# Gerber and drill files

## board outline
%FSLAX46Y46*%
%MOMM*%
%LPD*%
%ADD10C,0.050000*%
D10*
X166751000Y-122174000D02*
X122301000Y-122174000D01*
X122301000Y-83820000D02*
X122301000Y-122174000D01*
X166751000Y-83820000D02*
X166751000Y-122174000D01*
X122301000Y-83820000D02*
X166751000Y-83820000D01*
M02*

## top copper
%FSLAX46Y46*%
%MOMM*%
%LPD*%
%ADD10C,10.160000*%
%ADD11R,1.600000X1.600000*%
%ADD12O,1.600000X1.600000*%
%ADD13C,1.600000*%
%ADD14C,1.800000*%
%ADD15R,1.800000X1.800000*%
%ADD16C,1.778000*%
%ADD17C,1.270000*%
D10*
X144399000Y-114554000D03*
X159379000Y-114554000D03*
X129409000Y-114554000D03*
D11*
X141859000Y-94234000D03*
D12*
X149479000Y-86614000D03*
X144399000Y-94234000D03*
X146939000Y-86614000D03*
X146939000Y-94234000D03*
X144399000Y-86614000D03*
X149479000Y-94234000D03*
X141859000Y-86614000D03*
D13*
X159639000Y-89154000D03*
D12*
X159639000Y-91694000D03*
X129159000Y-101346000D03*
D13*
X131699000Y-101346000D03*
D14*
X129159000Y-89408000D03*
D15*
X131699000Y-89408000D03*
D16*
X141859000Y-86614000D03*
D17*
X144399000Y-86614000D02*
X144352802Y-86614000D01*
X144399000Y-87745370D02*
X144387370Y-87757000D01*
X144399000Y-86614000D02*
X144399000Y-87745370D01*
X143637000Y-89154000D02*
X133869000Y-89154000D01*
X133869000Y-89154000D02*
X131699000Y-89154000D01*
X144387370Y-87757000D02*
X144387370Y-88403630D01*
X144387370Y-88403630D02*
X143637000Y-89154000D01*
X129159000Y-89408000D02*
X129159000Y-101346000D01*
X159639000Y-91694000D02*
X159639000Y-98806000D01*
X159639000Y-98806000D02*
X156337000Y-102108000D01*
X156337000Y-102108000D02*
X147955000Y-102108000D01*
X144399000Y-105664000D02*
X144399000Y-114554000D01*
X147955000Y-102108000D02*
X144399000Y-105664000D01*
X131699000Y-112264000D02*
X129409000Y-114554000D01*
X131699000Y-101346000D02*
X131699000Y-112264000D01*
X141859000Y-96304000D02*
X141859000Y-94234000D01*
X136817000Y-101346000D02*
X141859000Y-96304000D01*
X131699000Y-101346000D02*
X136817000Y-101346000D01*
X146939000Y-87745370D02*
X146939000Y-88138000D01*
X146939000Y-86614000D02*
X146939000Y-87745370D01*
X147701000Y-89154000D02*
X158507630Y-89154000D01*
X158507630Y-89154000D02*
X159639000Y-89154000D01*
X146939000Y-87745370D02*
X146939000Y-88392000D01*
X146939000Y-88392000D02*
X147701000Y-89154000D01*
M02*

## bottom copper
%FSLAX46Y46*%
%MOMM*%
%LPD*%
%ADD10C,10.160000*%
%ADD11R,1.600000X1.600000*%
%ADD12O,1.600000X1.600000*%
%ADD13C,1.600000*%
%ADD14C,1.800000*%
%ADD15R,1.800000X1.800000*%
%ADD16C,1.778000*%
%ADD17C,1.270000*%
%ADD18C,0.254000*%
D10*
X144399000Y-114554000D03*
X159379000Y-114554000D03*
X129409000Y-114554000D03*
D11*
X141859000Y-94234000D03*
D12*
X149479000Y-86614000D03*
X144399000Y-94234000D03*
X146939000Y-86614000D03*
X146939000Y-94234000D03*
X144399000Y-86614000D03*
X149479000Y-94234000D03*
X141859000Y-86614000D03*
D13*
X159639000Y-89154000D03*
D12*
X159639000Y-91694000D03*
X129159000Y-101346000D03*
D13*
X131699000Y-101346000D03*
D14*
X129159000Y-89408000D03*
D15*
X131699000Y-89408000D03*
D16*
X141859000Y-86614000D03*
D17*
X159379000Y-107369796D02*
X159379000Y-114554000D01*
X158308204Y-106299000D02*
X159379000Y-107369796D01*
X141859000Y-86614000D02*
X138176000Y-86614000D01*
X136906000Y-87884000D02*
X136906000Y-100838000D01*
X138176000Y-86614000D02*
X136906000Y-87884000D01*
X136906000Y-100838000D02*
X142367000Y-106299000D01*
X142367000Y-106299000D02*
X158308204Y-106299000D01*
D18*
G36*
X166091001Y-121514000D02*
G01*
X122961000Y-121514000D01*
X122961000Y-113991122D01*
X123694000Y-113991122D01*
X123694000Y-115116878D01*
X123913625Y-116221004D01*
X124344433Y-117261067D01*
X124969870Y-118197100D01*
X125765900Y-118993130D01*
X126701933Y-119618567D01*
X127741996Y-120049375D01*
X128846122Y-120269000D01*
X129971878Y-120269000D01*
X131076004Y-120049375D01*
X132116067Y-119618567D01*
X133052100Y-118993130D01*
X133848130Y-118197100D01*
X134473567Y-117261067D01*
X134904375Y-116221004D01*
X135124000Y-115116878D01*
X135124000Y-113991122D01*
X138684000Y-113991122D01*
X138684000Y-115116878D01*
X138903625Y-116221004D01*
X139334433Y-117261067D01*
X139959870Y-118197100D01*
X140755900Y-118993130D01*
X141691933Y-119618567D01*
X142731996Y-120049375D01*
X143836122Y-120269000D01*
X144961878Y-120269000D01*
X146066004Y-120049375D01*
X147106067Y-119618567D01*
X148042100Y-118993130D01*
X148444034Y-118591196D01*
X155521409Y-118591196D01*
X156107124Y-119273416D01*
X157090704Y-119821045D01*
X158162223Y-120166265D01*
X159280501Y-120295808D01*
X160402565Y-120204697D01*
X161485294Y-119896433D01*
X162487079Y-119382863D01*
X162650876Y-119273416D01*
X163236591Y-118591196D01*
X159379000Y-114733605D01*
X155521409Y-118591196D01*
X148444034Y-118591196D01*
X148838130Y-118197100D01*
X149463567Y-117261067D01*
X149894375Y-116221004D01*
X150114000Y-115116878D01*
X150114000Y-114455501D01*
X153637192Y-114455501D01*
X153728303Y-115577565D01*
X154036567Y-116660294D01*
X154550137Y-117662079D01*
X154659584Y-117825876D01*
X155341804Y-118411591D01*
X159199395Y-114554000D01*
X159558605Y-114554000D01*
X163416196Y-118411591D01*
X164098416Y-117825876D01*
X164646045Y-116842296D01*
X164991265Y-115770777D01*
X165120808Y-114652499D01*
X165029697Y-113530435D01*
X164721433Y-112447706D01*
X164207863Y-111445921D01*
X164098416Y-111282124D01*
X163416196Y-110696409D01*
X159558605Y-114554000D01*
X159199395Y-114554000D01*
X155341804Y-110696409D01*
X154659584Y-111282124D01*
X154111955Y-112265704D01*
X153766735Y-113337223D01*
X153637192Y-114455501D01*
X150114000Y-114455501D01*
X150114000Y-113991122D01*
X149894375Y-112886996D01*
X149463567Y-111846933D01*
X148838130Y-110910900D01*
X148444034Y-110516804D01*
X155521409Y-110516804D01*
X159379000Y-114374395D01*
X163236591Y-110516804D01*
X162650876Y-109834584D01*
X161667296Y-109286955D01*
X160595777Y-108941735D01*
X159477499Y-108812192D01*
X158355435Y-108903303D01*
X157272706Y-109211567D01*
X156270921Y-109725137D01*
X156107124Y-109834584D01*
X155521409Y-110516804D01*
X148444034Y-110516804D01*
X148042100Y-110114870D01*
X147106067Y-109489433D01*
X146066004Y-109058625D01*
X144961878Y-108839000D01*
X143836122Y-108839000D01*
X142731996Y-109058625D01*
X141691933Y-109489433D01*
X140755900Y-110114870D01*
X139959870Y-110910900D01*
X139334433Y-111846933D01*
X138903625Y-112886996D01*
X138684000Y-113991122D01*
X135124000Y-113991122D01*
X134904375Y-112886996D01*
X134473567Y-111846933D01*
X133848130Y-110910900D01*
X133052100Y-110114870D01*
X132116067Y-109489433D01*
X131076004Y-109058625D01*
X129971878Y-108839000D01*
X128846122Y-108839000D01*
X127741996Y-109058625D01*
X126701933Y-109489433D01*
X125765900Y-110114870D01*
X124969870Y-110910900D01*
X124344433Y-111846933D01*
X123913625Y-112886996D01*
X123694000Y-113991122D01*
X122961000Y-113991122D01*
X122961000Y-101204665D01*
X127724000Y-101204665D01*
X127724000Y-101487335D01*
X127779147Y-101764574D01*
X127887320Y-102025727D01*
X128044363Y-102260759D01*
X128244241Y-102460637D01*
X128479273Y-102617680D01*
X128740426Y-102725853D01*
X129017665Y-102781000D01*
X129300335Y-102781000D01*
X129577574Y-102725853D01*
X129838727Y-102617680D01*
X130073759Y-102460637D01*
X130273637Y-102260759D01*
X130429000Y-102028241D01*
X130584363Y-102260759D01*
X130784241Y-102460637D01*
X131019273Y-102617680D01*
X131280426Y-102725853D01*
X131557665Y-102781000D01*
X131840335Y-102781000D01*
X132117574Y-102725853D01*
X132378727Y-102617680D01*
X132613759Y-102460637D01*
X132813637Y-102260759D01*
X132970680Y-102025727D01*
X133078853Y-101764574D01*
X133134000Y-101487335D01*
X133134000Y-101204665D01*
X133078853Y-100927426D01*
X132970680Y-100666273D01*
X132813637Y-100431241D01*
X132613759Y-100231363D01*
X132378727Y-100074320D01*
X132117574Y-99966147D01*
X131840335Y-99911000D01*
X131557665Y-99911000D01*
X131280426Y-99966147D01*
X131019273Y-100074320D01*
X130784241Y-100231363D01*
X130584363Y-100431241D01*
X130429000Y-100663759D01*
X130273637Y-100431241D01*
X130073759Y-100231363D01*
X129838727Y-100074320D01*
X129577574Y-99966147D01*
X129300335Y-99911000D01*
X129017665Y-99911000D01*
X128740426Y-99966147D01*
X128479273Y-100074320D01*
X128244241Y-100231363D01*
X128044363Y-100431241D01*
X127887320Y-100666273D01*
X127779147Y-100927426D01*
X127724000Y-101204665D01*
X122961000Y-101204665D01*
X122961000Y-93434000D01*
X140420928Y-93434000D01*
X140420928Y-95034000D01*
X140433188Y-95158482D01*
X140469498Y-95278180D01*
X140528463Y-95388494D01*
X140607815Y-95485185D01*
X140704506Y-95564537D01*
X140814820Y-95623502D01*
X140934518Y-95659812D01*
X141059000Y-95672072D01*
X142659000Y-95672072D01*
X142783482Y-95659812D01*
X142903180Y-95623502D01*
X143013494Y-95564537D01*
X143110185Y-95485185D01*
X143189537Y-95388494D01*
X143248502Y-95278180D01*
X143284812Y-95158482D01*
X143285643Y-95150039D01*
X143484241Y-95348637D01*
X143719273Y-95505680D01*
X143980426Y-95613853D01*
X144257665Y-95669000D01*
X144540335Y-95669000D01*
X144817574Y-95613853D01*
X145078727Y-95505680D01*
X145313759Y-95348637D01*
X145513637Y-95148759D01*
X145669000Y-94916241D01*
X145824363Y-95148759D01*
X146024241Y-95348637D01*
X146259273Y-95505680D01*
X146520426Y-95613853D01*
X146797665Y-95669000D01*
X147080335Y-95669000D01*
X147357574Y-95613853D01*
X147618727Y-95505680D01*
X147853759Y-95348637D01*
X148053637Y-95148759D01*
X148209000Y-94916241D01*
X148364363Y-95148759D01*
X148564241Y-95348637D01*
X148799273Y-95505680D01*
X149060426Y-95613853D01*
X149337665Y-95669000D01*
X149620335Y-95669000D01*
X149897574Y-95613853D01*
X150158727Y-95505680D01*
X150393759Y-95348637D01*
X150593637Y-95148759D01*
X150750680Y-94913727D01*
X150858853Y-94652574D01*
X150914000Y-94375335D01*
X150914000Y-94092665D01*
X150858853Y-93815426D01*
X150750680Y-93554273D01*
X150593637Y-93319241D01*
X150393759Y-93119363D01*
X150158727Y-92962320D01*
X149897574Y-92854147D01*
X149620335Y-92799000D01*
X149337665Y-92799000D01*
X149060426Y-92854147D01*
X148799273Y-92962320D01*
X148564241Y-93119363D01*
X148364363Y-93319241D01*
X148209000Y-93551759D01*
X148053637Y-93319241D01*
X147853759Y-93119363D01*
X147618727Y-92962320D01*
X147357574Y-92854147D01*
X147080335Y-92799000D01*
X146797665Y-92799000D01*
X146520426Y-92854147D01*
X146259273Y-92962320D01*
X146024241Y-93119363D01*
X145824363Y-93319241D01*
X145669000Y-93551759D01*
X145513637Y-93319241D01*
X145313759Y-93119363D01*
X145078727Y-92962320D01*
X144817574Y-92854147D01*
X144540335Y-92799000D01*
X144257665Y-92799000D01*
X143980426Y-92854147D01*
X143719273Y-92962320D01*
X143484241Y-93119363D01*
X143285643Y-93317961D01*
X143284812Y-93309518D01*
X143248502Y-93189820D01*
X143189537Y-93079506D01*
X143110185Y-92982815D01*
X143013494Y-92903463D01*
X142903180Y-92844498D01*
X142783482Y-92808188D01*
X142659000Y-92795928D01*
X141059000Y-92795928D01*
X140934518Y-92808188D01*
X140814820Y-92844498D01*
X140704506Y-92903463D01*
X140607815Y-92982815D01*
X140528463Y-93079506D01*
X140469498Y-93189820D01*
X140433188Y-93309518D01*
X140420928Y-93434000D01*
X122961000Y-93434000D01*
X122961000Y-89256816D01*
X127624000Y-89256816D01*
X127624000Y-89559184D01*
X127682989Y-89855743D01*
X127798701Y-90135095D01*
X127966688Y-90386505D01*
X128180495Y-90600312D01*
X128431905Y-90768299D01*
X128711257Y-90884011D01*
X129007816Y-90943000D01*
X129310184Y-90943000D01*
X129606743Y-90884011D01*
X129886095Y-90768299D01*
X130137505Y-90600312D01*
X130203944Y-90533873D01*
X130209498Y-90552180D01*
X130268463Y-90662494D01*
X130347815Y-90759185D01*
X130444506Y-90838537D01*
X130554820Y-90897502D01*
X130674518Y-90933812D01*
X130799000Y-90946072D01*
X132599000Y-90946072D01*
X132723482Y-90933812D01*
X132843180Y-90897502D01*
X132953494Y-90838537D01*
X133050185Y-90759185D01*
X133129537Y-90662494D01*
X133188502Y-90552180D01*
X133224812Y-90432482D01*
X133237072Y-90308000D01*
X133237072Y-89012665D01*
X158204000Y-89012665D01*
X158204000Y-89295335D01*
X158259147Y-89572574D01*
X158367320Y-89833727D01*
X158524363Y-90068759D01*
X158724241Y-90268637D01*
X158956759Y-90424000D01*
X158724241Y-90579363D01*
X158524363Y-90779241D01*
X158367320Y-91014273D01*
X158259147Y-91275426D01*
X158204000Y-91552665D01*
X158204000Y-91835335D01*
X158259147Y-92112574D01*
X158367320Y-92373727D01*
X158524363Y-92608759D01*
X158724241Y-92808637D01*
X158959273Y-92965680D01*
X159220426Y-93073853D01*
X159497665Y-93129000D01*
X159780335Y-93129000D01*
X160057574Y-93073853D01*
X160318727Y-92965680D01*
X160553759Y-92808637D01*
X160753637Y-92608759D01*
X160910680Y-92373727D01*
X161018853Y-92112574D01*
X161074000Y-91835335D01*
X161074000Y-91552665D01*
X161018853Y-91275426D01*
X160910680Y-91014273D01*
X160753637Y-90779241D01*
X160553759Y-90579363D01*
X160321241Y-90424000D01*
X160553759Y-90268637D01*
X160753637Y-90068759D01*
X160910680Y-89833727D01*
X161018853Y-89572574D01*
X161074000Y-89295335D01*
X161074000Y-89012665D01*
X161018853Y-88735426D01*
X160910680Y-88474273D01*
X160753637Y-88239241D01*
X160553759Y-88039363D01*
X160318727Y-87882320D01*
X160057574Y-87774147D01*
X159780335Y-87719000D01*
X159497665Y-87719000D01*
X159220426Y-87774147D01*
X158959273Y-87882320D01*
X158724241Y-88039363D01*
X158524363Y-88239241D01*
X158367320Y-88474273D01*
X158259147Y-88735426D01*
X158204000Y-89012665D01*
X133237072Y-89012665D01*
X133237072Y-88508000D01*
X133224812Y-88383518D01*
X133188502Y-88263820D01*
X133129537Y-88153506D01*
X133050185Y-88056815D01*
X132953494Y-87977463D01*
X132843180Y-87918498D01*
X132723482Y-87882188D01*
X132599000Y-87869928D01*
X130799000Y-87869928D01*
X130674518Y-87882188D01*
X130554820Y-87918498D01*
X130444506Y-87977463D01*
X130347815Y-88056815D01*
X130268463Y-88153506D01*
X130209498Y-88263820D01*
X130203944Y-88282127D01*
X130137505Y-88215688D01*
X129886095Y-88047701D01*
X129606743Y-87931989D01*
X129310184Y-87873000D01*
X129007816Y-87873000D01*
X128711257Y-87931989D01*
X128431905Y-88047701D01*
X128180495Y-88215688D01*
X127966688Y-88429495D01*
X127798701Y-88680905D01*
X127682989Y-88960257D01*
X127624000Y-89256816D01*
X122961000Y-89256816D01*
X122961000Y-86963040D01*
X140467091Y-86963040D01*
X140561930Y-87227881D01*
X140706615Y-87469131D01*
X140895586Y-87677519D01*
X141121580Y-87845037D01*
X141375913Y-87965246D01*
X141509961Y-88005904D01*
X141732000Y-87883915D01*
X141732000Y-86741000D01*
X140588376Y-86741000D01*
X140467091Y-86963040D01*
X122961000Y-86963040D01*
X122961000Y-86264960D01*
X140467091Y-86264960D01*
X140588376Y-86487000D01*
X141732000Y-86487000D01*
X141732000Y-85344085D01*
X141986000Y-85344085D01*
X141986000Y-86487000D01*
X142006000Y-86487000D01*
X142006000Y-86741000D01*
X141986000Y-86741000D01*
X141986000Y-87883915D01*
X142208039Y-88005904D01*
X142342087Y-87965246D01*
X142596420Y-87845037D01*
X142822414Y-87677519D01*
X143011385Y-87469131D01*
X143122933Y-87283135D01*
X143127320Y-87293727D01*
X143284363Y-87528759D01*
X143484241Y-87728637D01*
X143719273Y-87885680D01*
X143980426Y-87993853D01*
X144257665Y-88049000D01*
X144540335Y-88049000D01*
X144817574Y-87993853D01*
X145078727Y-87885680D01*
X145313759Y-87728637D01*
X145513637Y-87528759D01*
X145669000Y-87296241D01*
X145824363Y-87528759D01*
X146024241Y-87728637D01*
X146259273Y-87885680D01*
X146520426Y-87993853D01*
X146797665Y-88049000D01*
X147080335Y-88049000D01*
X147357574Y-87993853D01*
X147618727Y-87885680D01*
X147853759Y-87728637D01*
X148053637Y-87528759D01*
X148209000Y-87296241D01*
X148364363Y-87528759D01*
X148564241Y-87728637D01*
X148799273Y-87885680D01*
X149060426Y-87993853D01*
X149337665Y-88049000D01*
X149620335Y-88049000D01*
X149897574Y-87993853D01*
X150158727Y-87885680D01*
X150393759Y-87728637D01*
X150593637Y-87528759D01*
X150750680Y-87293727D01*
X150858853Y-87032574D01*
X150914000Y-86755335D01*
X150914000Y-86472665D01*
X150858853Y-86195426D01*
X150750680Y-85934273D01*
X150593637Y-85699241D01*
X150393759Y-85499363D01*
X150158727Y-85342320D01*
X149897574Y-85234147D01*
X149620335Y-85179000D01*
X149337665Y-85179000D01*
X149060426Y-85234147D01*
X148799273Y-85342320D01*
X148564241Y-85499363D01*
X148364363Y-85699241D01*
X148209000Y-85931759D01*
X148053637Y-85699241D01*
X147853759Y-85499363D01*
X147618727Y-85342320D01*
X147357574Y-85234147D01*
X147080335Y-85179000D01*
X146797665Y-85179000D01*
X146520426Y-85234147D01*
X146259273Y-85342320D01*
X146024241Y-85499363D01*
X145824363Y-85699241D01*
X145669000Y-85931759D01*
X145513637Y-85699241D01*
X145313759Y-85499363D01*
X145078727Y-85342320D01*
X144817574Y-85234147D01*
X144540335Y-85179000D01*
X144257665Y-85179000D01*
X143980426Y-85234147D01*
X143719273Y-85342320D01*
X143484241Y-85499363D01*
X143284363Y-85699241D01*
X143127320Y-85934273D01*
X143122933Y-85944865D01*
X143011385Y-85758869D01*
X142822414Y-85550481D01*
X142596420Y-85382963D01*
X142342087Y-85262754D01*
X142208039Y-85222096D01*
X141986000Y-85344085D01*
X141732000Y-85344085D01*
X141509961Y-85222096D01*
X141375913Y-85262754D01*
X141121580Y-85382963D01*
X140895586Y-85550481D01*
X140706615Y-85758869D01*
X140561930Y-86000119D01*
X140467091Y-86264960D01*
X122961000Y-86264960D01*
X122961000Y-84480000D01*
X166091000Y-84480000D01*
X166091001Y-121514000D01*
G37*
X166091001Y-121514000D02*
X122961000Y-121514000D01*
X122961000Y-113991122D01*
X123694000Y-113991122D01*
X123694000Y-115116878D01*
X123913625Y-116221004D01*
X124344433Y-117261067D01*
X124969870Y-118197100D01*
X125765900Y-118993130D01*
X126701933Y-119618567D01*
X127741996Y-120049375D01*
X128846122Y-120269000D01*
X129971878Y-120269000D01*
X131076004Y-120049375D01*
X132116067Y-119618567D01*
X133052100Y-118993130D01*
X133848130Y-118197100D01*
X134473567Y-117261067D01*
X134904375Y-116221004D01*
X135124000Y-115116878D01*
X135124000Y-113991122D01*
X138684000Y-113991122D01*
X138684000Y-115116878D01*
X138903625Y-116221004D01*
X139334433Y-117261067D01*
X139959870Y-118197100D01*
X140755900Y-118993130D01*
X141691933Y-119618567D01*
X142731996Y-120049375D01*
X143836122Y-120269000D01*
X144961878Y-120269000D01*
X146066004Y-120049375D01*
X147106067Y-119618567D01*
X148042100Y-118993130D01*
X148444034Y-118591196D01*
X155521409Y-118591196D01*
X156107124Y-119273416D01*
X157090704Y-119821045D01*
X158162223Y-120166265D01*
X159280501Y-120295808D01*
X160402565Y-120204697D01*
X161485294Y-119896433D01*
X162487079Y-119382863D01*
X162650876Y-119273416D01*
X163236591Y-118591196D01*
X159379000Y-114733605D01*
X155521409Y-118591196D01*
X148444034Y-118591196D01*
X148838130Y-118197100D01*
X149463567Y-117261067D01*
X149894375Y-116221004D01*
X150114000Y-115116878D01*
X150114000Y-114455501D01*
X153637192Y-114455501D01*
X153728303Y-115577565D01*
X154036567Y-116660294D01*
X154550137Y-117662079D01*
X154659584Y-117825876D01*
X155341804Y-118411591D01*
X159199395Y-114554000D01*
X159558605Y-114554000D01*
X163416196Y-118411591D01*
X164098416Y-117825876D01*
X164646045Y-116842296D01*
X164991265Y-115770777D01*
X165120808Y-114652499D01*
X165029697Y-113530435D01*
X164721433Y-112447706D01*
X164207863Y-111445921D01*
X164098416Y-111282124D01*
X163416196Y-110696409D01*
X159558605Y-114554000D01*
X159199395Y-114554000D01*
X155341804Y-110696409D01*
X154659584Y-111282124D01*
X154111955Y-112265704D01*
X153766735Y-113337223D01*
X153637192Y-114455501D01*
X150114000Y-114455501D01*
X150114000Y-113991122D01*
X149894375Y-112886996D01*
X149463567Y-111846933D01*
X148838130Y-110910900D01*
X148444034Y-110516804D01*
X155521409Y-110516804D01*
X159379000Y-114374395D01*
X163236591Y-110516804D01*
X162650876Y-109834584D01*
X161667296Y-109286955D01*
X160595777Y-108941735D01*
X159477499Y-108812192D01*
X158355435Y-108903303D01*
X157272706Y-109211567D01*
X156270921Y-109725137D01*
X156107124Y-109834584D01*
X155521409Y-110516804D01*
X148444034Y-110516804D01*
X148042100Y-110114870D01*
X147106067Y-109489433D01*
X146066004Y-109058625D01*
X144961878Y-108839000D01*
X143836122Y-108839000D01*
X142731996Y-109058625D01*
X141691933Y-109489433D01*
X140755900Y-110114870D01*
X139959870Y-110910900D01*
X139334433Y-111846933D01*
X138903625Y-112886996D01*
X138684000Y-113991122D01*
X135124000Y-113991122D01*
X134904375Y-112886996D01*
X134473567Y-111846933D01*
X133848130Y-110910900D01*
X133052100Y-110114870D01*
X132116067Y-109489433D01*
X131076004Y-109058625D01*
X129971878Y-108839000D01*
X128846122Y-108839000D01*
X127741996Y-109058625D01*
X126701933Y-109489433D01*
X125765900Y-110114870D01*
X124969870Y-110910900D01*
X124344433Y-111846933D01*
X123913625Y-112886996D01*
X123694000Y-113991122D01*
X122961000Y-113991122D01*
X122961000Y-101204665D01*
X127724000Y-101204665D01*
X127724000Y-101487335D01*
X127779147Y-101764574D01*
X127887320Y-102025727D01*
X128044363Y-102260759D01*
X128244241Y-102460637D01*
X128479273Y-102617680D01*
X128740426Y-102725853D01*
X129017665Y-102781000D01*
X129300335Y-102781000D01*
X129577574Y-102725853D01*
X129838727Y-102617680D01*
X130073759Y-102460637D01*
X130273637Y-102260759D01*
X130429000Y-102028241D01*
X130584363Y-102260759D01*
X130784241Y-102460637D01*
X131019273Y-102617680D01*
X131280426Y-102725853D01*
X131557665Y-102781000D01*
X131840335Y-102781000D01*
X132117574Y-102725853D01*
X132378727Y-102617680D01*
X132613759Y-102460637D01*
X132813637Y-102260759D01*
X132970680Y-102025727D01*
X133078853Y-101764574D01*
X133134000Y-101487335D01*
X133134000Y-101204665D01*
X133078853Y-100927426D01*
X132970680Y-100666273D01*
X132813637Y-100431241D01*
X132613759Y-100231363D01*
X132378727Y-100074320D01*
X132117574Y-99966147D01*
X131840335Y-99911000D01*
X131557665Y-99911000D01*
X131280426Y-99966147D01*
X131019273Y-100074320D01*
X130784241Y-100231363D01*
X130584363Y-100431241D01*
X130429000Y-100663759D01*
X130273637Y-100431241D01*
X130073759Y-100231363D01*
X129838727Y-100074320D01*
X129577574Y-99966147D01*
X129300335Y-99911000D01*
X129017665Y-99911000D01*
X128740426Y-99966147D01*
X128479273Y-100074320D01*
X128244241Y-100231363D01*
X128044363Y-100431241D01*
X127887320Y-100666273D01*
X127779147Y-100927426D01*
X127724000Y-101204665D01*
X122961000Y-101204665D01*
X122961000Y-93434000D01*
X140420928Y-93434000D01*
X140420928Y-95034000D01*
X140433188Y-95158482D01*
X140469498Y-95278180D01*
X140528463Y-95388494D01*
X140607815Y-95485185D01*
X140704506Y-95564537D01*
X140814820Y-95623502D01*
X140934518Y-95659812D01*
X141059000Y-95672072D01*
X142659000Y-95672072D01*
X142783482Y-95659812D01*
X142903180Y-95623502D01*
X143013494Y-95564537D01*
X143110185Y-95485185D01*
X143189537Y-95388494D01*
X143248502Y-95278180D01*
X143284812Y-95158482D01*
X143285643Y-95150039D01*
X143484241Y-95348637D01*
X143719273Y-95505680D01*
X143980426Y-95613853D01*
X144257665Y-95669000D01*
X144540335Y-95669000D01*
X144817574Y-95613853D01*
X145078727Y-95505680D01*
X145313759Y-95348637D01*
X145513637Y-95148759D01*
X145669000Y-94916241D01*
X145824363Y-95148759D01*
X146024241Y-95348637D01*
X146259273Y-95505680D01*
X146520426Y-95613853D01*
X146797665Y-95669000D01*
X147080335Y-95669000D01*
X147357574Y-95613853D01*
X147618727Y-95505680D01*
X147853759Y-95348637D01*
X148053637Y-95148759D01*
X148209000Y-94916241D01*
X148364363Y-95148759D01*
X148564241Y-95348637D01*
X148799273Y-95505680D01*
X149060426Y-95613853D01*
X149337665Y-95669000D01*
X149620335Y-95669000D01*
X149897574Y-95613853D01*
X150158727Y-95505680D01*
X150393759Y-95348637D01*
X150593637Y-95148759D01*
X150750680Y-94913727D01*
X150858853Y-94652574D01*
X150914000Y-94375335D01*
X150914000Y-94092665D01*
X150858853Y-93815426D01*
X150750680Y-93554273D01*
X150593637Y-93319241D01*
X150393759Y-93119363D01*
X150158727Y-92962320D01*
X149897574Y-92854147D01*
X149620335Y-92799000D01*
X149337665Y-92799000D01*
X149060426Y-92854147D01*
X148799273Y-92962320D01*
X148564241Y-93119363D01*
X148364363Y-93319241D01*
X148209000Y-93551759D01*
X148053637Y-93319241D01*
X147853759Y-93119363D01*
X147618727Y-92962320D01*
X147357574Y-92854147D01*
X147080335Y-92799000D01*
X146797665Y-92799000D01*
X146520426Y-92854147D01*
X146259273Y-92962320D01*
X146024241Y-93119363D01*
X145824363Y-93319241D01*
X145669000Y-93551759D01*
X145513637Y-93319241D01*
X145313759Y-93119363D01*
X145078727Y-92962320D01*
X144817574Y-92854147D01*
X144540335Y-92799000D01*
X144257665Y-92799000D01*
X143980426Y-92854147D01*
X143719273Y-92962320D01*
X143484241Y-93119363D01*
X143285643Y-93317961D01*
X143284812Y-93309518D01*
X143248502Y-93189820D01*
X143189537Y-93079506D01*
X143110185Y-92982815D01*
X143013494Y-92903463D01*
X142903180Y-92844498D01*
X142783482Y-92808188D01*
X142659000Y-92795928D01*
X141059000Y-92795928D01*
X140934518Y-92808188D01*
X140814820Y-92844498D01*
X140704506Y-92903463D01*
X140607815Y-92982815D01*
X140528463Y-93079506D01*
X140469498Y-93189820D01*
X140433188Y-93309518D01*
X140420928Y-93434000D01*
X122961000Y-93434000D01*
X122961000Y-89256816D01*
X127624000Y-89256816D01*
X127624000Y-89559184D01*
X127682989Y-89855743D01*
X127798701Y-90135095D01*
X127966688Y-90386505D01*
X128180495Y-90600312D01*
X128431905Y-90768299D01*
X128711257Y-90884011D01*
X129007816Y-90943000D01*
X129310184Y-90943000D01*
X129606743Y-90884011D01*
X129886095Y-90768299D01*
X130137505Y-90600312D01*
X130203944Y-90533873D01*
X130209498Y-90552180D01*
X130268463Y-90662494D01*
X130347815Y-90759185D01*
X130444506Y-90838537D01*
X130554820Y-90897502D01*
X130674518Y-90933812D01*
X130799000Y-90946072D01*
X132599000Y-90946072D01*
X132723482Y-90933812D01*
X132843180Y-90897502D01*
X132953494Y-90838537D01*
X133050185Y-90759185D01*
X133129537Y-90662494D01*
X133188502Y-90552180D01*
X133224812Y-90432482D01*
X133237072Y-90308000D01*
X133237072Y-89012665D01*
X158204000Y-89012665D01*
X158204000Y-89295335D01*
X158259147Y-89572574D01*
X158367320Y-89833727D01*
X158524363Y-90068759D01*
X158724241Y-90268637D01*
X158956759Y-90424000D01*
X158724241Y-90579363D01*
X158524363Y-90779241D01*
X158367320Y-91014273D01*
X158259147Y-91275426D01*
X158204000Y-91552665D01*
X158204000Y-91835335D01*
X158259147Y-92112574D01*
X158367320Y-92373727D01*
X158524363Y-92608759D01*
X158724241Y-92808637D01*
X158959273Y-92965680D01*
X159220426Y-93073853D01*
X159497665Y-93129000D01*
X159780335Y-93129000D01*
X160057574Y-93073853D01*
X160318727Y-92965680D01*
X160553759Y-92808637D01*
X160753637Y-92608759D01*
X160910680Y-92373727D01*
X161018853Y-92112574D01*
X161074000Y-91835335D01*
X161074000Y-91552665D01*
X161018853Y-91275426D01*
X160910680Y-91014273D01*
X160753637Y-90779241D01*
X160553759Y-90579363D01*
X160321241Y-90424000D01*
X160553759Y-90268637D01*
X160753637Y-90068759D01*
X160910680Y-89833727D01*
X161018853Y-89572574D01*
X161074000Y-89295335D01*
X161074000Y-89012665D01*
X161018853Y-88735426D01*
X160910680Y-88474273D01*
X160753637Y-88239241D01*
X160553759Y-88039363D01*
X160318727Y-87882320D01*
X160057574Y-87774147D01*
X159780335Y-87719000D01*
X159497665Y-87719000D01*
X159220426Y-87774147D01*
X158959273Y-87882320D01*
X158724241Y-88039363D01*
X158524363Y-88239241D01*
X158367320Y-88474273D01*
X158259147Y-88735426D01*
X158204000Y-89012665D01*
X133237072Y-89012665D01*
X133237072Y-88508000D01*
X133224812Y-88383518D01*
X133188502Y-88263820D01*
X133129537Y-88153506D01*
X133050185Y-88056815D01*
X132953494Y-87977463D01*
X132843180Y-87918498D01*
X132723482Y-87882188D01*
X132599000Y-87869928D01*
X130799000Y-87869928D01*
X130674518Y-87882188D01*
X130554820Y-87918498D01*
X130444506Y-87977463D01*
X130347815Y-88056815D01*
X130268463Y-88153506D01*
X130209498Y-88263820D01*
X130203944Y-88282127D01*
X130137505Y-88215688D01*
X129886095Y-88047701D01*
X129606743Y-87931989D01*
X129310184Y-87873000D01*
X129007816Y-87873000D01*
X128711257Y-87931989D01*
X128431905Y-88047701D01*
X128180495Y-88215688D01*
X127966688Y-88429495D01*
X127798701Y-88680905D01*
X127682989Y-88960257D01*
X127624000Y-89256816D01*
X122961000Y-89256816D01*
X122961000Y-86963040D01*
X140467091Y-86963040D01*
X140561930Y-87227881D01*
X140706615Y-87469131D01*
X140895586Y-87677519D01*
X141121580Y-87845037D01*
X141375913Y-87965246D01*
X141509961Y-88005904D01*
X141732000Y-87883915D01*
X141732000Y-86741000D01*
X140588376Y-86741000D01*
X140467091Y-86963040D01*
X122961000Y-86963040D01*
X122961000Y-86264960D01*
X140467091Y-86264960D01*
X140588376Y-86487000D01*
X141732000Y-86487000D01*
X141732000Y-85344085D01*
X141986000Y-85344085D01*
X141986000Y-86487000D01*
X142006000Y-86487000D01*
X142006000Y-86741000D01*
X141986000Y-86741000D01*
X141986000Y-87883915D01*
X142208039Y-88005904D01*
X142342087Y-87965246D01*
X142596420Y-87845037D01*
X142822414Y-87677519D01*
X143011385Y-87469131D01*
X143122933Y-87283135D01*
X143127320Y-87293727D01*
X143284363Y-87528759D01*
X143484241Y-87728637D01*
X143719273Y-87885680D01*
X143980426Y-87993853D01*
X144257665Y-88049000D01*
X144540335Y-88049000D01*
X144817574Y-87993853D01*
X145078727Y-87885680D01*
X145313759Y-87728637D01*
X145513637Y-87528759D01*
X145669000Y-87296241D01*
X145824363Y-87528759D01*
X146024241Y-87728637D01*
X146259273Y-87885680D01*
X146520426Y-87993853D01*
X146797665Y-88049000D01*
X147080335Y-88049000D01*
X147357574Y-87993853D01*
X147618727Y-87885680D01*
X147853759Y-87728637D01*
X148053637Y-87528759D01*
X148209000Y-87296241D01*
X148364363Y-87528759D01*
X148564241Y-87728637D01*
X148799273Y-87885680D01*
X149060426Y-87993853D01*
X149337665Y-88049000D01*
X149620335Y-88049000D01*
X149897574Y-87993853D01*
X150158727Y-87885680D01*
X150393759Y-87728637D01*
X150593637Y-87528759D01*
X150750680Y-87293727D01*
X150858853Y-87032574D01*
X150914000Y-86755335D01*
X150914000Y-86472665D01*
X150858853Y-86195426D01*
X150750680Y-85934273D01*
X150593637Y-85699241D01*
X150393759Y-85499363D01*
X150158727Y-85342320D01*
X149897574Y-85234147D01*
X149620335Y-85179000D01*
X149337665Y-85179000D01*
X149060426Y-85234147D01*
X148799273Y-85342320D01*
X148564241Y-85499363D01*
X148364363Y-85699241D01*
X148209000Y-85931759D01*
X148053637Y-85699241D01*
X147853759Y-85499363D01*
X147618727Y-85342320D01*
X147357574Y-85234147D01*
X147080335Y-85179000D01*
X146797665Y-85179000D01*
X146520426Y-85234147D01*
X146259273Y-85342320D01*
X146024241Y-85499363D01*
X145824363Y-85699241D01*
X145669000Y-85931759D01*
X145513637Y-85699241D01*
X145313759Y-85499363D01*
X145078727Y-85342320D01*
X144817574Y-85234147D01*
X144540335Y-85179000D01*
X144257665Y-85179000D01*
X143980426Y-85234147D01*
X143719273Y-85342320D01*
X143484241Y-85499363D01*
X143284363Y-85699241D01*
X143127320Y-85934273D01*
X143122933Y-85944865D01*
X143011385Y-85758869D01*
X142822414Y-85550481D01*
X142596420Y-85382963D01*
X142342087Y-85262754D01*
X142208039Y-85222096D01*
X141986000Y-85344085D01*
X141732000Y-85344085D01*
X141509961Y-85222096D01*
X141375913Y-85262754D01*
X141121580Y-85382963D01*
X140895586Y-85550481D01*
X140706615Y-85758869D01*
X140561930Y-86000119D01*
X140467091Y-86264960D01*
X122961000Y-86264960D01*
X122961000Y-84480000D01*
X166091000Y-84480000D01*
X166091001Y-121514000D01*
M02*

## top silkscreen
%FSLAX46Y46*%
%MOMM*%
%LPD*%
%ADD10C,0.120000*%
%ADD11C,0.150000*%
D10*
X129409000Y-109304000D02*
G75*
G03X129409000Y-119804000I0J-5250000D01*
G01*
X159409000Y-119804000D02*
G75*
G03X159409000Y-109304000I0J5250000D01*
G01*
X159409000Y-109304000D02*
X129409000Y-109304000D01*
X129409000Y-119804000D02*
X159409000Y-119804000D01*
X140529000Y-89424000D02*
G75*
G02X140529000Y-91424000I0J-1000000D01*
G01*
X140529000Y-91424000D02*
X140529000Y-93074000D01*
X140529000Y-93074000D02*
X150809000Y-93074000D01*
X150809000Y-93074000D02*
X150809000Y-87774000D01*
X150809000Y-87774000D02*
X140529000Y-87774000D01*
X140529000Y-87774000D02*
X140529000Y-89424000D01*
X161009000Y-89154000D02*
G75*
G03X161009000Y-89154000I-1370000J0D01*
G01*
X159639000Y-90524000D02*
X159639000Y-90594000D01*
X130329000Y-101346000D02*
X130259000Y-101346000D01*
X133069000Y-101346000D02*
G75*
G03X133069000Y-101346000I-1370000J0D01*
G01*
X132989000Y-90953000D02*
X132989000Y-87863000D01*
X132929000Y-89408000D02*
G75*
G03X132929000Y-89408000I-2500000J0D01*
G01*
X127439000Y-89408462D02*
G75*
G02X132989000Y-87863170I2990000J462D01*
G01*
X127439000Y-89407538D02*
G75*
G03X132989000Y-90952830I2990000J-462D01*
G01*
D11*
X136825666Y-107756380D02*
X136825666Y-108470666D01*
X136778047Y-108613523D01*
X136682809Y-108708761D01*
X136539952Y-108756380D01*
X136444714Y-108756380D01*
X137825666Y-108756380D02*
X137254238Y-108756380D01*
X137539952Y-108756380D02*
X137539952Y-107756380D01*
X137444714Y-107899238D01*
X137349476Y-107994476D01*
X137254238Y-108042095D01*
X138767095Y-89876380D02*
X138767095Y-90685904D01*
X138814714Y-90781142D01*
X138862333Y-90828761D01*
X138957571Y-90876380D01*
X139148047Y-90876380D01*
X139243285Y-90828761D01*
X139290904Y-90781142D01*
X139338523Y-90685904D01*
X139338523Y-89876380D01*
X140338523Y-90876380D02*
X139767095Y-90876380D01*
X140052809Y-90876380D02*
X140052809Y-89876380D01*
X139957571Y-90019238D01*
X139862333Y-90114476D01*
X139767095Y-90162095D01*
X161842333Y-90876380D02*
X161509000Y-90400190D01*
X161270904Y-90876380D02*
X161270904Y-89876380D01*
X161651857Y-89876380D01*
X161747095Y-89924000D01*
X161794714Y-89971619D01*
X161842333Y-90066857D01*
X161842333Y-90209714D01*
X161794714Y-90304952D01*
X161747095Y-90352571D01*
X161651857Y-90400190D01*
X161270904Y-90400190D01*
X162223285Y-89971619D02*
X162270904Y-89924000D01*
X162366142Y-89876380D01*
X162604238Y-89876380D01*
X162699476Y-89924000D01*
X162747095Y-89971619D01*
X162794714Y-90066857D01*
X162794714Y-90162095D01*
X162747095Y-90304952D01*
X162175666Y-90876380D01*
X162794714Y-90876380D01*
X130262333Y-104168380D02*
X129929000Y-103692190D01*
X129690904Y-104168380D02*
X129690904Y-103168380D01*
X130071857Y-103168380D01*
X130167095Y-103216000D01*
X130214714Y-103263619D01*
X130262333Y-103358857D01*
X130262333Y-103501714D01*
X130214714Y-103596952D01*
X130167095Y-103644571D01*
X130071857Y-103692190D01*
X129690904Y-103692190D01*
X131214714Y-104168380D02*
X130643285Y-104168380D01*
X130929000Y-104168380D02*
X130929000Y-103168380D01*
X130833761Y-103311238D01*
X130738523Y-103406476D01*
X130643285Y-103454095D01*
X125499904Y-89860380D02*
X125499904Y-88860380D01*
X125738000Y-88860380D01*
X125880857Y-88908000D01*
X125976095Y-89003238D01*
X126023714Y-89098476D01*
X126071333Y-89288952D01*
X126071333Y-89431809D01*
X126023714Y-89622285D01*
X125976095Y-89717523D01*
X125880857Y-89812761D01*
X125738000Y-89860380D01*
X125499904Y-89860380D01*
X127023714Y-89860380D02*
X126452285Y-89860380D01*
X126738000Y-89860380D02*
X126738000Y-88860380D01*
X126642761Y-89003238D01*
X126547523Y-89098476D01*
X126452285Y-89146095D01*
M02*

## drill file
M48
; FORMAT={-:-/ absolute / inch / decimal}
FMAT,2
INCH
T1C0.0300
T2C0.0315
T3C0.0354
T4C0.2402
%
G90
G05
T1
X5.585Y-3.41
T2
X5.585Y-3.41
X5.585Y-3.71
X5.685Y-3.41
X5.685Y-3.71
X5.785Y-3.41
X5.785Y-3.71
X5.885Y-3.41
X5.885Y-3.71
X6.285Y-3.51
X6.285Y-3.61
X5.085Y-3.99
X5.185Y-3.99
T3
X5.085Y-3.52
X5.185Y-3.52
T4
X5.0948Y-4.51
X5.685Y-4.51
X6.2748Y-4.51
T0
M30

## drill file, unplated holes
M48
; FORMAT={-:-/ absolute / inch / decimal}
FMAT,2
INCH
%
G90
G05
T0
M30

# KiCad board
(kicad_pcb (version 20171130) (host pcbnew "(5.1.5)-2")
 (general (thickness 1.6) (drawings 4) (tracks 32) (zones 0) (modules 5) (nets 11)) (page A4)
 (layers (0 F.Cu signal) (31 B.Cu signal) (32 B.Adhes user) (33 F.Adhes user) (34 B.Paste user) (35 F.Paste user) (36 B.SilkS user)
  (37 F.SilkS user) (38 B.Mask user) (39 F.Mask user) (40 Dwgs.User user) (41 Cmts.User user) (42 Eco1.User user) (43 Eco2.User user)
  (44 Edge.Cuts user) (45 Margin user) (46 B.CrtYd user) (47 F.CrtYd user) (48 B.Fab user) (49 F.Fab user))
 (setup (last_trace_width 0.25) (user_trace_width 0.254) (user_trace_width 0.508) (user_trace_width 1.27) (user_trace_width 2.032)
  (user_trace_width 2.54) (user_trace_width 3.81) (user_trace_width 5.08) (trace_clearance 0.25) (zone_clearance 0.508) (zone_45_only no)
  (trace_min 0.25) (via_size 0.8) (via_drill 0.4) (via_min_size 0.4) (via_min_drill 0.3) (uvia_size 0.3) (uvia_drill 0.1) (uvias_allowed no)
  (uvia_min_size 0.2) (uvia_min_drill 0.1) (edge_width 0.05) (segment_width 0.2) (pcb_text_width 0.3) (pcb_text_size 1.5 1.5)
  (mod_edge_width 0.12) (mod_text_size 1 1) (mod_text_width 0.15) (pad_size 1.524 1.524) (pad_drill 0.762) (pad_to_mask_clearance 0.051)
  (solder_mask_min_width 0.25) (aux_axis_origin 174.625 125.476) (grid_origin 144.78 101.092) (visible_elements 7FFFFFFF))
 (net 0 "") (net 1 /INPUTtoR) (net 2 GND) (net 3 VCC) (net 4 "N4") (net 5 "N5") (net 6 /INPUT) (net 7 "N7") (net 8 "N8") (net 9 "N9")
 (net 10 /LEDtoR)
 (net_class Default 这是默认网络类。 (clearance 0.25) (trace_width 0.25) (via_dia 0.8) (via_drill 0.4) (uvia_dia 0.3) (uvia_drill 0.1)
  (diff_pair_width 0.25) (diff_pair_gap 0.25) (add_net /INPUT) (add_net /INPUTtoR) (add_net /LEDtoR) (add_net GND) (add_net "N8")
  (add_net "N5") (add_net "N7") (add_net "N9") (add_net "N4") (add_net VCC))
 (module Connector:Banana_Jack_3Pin (layer F.Cu) (at 129.409 114.554)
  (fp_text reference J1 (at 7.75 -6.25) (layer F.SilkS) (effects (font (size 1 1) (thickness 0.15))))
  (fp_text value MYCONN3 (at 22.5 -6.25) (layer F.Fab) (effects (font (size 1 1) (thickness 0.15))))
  (fp_arc (start 0 0) (end 0 5.25) (angle 180) (layer F.SilkS) (width 0.12))
  (fp_arc (start 30 0) (end 30 -5.25) (angle 180) (layer F.SilkS) (width 0.12))
  (fp_line (start 30 -5.25) (end 0 -5.25) (layer F.SilkS) (width 0.12))
  (fp_line (start 0 5.25) (end 30 5.25) (layer F.SilkS) (width 0.12))
  (pad 2 thru_hole circle (at 14.99 0) (size 10.16 10.16) (drill 6.1) (layers *.Cu *.Mask) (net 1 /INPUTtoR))
  (pad 3 thru_hole circle (at 29.97 0) (size 10.16 10.16) (drill 6.1) (layers *.Cu *.Mask) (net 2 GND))
  (pad 1 thru_hole circle (at 0 0) (size 10.16 10.16) (drill 6.1) (layers *.Cu *.Mask) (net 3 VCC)))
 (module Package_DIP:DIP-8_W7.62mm (layer F.Cu) (at 141.859 94.234 90)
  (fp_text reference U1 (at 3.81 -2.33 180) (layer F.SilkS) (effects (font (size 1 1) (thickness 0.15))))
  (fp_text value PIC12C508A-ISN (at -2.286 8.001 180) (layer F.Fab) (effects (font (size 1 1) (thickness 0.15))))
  (fp_arc (start 3.81 -1.33) (end 2.81 -1.33) (angle -180) (layer F.SilkS) (width 0.12))
  (fp_line (start 2.81 -1.33) (end 1.16 -1.33) (layer F.SilkS) (width 0.12))
  (fp_line (start 1.16 -1.33) (end 1.16 8.95) (layer F.SilkS) (width 0.12))
  (fp_line (start 1.16 8.95) (end 6.46 8.95) (layer F.SilkS) (width 0.12))
  (fp_line (start 6.46 8.95) (end 6.46 -1.33) (layer F.SilkS) (width 0.12))
  (fp_line (start 6.46 -1.33) (end 4.81 -1.33) (layer F.SilkS) (width 0.12))
  (pad 1 thru_hole rect (at 0 0 90) (size 1.6 1.6) (drill 0.8) (layers *.Cu *.Mask) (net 3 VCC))
  (pad 5 thru_hole oval (at 7.62 7.62 90) (size 1.6 1.6) (drill 0.8) (layers *.Cu *.Mask) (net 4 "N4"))
  (pad 2 thru_hole oval (at 0 2.54 90) (size 1.6 1.6) (drill 0.8) (layers *.Cu *.Mask) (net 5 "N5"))
  (pad 6 thru_hole oval (at 7.62 5.08 90) (size 1.6 1.6) (drill 0.8) (layers *.Cu *.Mask) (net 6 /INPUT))
  (pad 3 thru_hole oval (at 0 5.08 90) (size 1.6 1.6) (drill 0.8) (layers *.Cu *.Mask) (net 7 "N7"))
  (pad 7 thru_hole oval (at 7.62 2.54 90) (size 1.6 1.6) (drill 0.8) (layers *.Cu *.Mask) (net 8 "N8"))
  (pad 4 thru_hole oval (at 0 7.62 90) (size 1.6 1.6) (drill 0.8) (layers *.Cu *.Mask) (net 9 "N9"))
  (pad 8 thru_hole oval (at 7.62 0 90) (size 1.6 1.6) (drill 0.8) (layers *.Cu *.Mask) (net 2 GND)))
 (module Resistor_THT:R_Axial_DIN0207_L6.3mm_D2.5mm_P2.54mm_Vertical (layer F.Cu) (at 159.639 89.154 270)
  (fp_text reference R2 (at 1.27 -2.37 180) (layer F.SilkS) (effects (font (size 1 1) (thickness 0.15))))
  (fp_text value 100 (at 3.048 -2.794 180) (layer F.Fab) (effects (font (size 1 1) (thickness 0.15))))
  (fp_circle (center 0 0) (end 1.37 0) (layer F.SilkS) (width 0.12))
  (fp_line (start 1.37 0) (end 1.44 0) (layer F.SilkS) (width 0.12))
  (pad 1 thru_hole circle (at 0 0 270) (size 1.6 1.6) (drill 0.8) (layers *.Cu *.Mask) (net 6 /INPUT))
  (pad 2 thru_hole oval (at 2.54 0 270) (size 1.6 1.6) (drill 0.8) (layers *.Cu *.Mask) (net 1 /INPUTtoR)))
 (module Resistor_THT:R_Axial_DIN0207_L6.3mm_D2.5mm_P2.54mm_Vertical (layer F.Cu) (at 131.699 101.346 180)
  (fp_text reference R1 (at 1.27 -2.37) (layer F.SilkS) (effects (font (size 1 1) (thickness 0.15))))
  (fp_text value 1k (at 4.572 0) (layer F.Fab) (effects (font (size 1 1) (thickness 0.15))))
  (fp_line (start 1.37 0) (end 1.44 0) (layer F.SilkS) (width 0.12))
  (fp_circle (center 0 0) (end 1.37 0) (layer F.SilkS) (width 0.12))
  (pad 2 thru_hole oval (at 2.54 0 180) (size 1.6 1.6) (drill 0.8) (layers *.Cu *.Mask) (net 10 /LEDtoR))
  (pad 1 thru_hole circle (at 0 0 180) (size 1.6 1.6) (drill 0.8) (layers *.Cu *.Mask) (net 3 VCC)))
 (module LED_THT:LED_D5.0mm (layer F.Cu) (at 131.699 89.408 180)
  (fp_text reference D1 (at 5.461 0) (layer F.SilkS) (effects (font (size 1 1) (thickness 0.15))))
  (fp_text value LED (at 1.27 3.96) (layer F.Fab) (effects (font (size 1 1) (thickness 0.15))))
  (fp_line (start -1.29 -1.545) (end -1.29 1.545) (layer F.SilkS) (width 0.12))
  (fp_circle (center 1.27 0) (end 3.77 0) (layer F.SilkS) (width 0.12))
  (fp_arc (start 1.27 0) (end -1.29 1.54483) (angle -148.9) (layer F.SilkS) (width 0.12))
  (fp_arc (start 1.27 0) (end -1.29 -1.54483) (angle 148.9) (layer F.SilkS) (width 0.12))
  (pad 2 thru_hole circle (at 2.54 0 180) (size 1.8 1.8) (drill 0.9) (layers *.Cu *.Mask) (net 10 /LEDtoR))
  (pad 1 thru_hole rect (at 0 0 180) (size 1.8 1.8) (drill 0.9) (layers *.Cu *.Mask) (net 8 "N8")))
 (gr_line (start 166.751 122.174) (end 122.301 122.174) (layer Edge.Cuts) (width 0.05))
 (gr_line (start 122.301 83.82) (end 122.301 122.174) (layer Edge.Cuts) (width 0.05))
 (gr_line (start 166.751 83.82) (end 166.751 122.174) (layer Edge.Cuts) (width 0.05))
 (gr_line (start 122.301 83.82) (end 166.751 83.82) (layer Edge.Cuts) (width 0.05))
 (segment (start 144.399 86.614) (end 144.352802 86.614) (width 1.27) (layer F.Cu) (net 8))
 (segment (start 144.399 87.74537) (end 144.38737 87.757) (width 1.27) (layer F.Cu) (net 8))
 (segment (start 144.399 86.614) (end 144.399 87.74537) (width 1.27) (layer F.Cu) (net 8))
 (segment (start 143.637 89.154) (end 133.869 89.154) (width 1.27) (layer F.Cu) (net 8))
 (segment (start 133.869 89.154) (end 131.699 89.154) (width 1.27) (layer F.Cu) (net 8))
 (segment (start 144.38737 87.757) (end 144.38737 88.40363) (width 1.27) (layer F.Cu) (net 8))
 (segment (start 144.38737 88.40363) (end 143.637 89.154) (width 1.27) (layer F.Cu) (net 8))
 (segment (start 129.159 89.408) (end 129.159 101.346) (width 1.27) (layer F.Cu) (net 10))
 (segment (start 159.639 91.694) (end 159.639 98.806) (width 1.27) (layer F.Cu) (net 1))
 (segment (start 159.639 98.806) (end 156.337 102.108) (width 1.27) (layer F.Cu) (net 1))
 (segment (start 156.337 102.108) (end 147.955 102.108) (width 1.27) (layer F.Cu) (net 1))
 (segment (start 144.399 105.664) (end 144.399 114.554) (width 1.27) (layer F.Cu) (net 1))
 (segment (start 147.955 102.108) (end 144.399 105.664) (width 1.27) (layer F.Cu) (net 1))
 (via (at 141.859 86.614) (size 1.778) (drill 0.762) (layers F.Cu B.Cu) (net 2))
 (segment (start 159.379 107.369796) (end 159.379 114.554) (width 1.27) (layer B.Cu) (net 2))
 (segment (start 158.308204 106.299) (end 159.379 107.369796) (width 1.27) (layer B.Cu) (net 2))
 (segment (start 141.859 86.614) (end 138.176 86.614) (width 1.27) (layer B.Cu) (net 2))
 (segment (start 136.906 87.884) (end 136.906 100.838) (width 1.27) (layer B.Cu) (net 2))
 (segment (start 138.176 86.614) (end 136.906 87.884) (width 1.27) (layer B.Cu) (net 2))
 (segment (start 136.906 100.838) (end 142.367 106.299) (width 1.27) (layer B.Cu) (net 2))
 (segment (start 142.367 106.299) (end 158.308204 106.299) (width 1.27) (layer B.Cu) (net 2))
 (segment (start 131.699 112.264) (end 129.409 114.554) (width 1.27) (layer F.Cu) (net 3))
 (segment (start 131.699 101.346) (end 131.699 112.264) (width 1.27) (layer F.Cu) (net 3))
 (segment (start 141.859 96.304) (end 141.859 94.234) (width 1.27) (layer F.Cu) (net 3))
 (segment (start 136.817 101.346) (end 141.859 96.304) (width 1.27) (layer F.Cu) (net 3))
 (segment (start 131.699 101.346) (end 136.817 101.346) (width 1.27) (layer F.Cu) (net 3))
 (segment (start 146.939 87.74537) (end 146.939 88.138) (width 1.27) (layer F.Cu) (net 6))
 (segment (start 146.939 86.614) (end 146.939 87.74537) (width 1.27) (layer F.Cu) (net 6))
 (segment (start 147.701 89.154) (end 158.50763 89.154) (width 1.27) (layer F.Cu) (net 6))
 (segment (start 158.50763 89.154) (end 159.639 89.154) (width 1.27) (layer F.Cu) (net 6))
 (segment (start 146.939 87.74537) (end 146.939 88.392) (width 1.27) (layer F.Cu) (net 6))
 (segment (start 146.939 88.392) (end 147.701 89.154) (width 1.27) (layer F.Cu) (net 6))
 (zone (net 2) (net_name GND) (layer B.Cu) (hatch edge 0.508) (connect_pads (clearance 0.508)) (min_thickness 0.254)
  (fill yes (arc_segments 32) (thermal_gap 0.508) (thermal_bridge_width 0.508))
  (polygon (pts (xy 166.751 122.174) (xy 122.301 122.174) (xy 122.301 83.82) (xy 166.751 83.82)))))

